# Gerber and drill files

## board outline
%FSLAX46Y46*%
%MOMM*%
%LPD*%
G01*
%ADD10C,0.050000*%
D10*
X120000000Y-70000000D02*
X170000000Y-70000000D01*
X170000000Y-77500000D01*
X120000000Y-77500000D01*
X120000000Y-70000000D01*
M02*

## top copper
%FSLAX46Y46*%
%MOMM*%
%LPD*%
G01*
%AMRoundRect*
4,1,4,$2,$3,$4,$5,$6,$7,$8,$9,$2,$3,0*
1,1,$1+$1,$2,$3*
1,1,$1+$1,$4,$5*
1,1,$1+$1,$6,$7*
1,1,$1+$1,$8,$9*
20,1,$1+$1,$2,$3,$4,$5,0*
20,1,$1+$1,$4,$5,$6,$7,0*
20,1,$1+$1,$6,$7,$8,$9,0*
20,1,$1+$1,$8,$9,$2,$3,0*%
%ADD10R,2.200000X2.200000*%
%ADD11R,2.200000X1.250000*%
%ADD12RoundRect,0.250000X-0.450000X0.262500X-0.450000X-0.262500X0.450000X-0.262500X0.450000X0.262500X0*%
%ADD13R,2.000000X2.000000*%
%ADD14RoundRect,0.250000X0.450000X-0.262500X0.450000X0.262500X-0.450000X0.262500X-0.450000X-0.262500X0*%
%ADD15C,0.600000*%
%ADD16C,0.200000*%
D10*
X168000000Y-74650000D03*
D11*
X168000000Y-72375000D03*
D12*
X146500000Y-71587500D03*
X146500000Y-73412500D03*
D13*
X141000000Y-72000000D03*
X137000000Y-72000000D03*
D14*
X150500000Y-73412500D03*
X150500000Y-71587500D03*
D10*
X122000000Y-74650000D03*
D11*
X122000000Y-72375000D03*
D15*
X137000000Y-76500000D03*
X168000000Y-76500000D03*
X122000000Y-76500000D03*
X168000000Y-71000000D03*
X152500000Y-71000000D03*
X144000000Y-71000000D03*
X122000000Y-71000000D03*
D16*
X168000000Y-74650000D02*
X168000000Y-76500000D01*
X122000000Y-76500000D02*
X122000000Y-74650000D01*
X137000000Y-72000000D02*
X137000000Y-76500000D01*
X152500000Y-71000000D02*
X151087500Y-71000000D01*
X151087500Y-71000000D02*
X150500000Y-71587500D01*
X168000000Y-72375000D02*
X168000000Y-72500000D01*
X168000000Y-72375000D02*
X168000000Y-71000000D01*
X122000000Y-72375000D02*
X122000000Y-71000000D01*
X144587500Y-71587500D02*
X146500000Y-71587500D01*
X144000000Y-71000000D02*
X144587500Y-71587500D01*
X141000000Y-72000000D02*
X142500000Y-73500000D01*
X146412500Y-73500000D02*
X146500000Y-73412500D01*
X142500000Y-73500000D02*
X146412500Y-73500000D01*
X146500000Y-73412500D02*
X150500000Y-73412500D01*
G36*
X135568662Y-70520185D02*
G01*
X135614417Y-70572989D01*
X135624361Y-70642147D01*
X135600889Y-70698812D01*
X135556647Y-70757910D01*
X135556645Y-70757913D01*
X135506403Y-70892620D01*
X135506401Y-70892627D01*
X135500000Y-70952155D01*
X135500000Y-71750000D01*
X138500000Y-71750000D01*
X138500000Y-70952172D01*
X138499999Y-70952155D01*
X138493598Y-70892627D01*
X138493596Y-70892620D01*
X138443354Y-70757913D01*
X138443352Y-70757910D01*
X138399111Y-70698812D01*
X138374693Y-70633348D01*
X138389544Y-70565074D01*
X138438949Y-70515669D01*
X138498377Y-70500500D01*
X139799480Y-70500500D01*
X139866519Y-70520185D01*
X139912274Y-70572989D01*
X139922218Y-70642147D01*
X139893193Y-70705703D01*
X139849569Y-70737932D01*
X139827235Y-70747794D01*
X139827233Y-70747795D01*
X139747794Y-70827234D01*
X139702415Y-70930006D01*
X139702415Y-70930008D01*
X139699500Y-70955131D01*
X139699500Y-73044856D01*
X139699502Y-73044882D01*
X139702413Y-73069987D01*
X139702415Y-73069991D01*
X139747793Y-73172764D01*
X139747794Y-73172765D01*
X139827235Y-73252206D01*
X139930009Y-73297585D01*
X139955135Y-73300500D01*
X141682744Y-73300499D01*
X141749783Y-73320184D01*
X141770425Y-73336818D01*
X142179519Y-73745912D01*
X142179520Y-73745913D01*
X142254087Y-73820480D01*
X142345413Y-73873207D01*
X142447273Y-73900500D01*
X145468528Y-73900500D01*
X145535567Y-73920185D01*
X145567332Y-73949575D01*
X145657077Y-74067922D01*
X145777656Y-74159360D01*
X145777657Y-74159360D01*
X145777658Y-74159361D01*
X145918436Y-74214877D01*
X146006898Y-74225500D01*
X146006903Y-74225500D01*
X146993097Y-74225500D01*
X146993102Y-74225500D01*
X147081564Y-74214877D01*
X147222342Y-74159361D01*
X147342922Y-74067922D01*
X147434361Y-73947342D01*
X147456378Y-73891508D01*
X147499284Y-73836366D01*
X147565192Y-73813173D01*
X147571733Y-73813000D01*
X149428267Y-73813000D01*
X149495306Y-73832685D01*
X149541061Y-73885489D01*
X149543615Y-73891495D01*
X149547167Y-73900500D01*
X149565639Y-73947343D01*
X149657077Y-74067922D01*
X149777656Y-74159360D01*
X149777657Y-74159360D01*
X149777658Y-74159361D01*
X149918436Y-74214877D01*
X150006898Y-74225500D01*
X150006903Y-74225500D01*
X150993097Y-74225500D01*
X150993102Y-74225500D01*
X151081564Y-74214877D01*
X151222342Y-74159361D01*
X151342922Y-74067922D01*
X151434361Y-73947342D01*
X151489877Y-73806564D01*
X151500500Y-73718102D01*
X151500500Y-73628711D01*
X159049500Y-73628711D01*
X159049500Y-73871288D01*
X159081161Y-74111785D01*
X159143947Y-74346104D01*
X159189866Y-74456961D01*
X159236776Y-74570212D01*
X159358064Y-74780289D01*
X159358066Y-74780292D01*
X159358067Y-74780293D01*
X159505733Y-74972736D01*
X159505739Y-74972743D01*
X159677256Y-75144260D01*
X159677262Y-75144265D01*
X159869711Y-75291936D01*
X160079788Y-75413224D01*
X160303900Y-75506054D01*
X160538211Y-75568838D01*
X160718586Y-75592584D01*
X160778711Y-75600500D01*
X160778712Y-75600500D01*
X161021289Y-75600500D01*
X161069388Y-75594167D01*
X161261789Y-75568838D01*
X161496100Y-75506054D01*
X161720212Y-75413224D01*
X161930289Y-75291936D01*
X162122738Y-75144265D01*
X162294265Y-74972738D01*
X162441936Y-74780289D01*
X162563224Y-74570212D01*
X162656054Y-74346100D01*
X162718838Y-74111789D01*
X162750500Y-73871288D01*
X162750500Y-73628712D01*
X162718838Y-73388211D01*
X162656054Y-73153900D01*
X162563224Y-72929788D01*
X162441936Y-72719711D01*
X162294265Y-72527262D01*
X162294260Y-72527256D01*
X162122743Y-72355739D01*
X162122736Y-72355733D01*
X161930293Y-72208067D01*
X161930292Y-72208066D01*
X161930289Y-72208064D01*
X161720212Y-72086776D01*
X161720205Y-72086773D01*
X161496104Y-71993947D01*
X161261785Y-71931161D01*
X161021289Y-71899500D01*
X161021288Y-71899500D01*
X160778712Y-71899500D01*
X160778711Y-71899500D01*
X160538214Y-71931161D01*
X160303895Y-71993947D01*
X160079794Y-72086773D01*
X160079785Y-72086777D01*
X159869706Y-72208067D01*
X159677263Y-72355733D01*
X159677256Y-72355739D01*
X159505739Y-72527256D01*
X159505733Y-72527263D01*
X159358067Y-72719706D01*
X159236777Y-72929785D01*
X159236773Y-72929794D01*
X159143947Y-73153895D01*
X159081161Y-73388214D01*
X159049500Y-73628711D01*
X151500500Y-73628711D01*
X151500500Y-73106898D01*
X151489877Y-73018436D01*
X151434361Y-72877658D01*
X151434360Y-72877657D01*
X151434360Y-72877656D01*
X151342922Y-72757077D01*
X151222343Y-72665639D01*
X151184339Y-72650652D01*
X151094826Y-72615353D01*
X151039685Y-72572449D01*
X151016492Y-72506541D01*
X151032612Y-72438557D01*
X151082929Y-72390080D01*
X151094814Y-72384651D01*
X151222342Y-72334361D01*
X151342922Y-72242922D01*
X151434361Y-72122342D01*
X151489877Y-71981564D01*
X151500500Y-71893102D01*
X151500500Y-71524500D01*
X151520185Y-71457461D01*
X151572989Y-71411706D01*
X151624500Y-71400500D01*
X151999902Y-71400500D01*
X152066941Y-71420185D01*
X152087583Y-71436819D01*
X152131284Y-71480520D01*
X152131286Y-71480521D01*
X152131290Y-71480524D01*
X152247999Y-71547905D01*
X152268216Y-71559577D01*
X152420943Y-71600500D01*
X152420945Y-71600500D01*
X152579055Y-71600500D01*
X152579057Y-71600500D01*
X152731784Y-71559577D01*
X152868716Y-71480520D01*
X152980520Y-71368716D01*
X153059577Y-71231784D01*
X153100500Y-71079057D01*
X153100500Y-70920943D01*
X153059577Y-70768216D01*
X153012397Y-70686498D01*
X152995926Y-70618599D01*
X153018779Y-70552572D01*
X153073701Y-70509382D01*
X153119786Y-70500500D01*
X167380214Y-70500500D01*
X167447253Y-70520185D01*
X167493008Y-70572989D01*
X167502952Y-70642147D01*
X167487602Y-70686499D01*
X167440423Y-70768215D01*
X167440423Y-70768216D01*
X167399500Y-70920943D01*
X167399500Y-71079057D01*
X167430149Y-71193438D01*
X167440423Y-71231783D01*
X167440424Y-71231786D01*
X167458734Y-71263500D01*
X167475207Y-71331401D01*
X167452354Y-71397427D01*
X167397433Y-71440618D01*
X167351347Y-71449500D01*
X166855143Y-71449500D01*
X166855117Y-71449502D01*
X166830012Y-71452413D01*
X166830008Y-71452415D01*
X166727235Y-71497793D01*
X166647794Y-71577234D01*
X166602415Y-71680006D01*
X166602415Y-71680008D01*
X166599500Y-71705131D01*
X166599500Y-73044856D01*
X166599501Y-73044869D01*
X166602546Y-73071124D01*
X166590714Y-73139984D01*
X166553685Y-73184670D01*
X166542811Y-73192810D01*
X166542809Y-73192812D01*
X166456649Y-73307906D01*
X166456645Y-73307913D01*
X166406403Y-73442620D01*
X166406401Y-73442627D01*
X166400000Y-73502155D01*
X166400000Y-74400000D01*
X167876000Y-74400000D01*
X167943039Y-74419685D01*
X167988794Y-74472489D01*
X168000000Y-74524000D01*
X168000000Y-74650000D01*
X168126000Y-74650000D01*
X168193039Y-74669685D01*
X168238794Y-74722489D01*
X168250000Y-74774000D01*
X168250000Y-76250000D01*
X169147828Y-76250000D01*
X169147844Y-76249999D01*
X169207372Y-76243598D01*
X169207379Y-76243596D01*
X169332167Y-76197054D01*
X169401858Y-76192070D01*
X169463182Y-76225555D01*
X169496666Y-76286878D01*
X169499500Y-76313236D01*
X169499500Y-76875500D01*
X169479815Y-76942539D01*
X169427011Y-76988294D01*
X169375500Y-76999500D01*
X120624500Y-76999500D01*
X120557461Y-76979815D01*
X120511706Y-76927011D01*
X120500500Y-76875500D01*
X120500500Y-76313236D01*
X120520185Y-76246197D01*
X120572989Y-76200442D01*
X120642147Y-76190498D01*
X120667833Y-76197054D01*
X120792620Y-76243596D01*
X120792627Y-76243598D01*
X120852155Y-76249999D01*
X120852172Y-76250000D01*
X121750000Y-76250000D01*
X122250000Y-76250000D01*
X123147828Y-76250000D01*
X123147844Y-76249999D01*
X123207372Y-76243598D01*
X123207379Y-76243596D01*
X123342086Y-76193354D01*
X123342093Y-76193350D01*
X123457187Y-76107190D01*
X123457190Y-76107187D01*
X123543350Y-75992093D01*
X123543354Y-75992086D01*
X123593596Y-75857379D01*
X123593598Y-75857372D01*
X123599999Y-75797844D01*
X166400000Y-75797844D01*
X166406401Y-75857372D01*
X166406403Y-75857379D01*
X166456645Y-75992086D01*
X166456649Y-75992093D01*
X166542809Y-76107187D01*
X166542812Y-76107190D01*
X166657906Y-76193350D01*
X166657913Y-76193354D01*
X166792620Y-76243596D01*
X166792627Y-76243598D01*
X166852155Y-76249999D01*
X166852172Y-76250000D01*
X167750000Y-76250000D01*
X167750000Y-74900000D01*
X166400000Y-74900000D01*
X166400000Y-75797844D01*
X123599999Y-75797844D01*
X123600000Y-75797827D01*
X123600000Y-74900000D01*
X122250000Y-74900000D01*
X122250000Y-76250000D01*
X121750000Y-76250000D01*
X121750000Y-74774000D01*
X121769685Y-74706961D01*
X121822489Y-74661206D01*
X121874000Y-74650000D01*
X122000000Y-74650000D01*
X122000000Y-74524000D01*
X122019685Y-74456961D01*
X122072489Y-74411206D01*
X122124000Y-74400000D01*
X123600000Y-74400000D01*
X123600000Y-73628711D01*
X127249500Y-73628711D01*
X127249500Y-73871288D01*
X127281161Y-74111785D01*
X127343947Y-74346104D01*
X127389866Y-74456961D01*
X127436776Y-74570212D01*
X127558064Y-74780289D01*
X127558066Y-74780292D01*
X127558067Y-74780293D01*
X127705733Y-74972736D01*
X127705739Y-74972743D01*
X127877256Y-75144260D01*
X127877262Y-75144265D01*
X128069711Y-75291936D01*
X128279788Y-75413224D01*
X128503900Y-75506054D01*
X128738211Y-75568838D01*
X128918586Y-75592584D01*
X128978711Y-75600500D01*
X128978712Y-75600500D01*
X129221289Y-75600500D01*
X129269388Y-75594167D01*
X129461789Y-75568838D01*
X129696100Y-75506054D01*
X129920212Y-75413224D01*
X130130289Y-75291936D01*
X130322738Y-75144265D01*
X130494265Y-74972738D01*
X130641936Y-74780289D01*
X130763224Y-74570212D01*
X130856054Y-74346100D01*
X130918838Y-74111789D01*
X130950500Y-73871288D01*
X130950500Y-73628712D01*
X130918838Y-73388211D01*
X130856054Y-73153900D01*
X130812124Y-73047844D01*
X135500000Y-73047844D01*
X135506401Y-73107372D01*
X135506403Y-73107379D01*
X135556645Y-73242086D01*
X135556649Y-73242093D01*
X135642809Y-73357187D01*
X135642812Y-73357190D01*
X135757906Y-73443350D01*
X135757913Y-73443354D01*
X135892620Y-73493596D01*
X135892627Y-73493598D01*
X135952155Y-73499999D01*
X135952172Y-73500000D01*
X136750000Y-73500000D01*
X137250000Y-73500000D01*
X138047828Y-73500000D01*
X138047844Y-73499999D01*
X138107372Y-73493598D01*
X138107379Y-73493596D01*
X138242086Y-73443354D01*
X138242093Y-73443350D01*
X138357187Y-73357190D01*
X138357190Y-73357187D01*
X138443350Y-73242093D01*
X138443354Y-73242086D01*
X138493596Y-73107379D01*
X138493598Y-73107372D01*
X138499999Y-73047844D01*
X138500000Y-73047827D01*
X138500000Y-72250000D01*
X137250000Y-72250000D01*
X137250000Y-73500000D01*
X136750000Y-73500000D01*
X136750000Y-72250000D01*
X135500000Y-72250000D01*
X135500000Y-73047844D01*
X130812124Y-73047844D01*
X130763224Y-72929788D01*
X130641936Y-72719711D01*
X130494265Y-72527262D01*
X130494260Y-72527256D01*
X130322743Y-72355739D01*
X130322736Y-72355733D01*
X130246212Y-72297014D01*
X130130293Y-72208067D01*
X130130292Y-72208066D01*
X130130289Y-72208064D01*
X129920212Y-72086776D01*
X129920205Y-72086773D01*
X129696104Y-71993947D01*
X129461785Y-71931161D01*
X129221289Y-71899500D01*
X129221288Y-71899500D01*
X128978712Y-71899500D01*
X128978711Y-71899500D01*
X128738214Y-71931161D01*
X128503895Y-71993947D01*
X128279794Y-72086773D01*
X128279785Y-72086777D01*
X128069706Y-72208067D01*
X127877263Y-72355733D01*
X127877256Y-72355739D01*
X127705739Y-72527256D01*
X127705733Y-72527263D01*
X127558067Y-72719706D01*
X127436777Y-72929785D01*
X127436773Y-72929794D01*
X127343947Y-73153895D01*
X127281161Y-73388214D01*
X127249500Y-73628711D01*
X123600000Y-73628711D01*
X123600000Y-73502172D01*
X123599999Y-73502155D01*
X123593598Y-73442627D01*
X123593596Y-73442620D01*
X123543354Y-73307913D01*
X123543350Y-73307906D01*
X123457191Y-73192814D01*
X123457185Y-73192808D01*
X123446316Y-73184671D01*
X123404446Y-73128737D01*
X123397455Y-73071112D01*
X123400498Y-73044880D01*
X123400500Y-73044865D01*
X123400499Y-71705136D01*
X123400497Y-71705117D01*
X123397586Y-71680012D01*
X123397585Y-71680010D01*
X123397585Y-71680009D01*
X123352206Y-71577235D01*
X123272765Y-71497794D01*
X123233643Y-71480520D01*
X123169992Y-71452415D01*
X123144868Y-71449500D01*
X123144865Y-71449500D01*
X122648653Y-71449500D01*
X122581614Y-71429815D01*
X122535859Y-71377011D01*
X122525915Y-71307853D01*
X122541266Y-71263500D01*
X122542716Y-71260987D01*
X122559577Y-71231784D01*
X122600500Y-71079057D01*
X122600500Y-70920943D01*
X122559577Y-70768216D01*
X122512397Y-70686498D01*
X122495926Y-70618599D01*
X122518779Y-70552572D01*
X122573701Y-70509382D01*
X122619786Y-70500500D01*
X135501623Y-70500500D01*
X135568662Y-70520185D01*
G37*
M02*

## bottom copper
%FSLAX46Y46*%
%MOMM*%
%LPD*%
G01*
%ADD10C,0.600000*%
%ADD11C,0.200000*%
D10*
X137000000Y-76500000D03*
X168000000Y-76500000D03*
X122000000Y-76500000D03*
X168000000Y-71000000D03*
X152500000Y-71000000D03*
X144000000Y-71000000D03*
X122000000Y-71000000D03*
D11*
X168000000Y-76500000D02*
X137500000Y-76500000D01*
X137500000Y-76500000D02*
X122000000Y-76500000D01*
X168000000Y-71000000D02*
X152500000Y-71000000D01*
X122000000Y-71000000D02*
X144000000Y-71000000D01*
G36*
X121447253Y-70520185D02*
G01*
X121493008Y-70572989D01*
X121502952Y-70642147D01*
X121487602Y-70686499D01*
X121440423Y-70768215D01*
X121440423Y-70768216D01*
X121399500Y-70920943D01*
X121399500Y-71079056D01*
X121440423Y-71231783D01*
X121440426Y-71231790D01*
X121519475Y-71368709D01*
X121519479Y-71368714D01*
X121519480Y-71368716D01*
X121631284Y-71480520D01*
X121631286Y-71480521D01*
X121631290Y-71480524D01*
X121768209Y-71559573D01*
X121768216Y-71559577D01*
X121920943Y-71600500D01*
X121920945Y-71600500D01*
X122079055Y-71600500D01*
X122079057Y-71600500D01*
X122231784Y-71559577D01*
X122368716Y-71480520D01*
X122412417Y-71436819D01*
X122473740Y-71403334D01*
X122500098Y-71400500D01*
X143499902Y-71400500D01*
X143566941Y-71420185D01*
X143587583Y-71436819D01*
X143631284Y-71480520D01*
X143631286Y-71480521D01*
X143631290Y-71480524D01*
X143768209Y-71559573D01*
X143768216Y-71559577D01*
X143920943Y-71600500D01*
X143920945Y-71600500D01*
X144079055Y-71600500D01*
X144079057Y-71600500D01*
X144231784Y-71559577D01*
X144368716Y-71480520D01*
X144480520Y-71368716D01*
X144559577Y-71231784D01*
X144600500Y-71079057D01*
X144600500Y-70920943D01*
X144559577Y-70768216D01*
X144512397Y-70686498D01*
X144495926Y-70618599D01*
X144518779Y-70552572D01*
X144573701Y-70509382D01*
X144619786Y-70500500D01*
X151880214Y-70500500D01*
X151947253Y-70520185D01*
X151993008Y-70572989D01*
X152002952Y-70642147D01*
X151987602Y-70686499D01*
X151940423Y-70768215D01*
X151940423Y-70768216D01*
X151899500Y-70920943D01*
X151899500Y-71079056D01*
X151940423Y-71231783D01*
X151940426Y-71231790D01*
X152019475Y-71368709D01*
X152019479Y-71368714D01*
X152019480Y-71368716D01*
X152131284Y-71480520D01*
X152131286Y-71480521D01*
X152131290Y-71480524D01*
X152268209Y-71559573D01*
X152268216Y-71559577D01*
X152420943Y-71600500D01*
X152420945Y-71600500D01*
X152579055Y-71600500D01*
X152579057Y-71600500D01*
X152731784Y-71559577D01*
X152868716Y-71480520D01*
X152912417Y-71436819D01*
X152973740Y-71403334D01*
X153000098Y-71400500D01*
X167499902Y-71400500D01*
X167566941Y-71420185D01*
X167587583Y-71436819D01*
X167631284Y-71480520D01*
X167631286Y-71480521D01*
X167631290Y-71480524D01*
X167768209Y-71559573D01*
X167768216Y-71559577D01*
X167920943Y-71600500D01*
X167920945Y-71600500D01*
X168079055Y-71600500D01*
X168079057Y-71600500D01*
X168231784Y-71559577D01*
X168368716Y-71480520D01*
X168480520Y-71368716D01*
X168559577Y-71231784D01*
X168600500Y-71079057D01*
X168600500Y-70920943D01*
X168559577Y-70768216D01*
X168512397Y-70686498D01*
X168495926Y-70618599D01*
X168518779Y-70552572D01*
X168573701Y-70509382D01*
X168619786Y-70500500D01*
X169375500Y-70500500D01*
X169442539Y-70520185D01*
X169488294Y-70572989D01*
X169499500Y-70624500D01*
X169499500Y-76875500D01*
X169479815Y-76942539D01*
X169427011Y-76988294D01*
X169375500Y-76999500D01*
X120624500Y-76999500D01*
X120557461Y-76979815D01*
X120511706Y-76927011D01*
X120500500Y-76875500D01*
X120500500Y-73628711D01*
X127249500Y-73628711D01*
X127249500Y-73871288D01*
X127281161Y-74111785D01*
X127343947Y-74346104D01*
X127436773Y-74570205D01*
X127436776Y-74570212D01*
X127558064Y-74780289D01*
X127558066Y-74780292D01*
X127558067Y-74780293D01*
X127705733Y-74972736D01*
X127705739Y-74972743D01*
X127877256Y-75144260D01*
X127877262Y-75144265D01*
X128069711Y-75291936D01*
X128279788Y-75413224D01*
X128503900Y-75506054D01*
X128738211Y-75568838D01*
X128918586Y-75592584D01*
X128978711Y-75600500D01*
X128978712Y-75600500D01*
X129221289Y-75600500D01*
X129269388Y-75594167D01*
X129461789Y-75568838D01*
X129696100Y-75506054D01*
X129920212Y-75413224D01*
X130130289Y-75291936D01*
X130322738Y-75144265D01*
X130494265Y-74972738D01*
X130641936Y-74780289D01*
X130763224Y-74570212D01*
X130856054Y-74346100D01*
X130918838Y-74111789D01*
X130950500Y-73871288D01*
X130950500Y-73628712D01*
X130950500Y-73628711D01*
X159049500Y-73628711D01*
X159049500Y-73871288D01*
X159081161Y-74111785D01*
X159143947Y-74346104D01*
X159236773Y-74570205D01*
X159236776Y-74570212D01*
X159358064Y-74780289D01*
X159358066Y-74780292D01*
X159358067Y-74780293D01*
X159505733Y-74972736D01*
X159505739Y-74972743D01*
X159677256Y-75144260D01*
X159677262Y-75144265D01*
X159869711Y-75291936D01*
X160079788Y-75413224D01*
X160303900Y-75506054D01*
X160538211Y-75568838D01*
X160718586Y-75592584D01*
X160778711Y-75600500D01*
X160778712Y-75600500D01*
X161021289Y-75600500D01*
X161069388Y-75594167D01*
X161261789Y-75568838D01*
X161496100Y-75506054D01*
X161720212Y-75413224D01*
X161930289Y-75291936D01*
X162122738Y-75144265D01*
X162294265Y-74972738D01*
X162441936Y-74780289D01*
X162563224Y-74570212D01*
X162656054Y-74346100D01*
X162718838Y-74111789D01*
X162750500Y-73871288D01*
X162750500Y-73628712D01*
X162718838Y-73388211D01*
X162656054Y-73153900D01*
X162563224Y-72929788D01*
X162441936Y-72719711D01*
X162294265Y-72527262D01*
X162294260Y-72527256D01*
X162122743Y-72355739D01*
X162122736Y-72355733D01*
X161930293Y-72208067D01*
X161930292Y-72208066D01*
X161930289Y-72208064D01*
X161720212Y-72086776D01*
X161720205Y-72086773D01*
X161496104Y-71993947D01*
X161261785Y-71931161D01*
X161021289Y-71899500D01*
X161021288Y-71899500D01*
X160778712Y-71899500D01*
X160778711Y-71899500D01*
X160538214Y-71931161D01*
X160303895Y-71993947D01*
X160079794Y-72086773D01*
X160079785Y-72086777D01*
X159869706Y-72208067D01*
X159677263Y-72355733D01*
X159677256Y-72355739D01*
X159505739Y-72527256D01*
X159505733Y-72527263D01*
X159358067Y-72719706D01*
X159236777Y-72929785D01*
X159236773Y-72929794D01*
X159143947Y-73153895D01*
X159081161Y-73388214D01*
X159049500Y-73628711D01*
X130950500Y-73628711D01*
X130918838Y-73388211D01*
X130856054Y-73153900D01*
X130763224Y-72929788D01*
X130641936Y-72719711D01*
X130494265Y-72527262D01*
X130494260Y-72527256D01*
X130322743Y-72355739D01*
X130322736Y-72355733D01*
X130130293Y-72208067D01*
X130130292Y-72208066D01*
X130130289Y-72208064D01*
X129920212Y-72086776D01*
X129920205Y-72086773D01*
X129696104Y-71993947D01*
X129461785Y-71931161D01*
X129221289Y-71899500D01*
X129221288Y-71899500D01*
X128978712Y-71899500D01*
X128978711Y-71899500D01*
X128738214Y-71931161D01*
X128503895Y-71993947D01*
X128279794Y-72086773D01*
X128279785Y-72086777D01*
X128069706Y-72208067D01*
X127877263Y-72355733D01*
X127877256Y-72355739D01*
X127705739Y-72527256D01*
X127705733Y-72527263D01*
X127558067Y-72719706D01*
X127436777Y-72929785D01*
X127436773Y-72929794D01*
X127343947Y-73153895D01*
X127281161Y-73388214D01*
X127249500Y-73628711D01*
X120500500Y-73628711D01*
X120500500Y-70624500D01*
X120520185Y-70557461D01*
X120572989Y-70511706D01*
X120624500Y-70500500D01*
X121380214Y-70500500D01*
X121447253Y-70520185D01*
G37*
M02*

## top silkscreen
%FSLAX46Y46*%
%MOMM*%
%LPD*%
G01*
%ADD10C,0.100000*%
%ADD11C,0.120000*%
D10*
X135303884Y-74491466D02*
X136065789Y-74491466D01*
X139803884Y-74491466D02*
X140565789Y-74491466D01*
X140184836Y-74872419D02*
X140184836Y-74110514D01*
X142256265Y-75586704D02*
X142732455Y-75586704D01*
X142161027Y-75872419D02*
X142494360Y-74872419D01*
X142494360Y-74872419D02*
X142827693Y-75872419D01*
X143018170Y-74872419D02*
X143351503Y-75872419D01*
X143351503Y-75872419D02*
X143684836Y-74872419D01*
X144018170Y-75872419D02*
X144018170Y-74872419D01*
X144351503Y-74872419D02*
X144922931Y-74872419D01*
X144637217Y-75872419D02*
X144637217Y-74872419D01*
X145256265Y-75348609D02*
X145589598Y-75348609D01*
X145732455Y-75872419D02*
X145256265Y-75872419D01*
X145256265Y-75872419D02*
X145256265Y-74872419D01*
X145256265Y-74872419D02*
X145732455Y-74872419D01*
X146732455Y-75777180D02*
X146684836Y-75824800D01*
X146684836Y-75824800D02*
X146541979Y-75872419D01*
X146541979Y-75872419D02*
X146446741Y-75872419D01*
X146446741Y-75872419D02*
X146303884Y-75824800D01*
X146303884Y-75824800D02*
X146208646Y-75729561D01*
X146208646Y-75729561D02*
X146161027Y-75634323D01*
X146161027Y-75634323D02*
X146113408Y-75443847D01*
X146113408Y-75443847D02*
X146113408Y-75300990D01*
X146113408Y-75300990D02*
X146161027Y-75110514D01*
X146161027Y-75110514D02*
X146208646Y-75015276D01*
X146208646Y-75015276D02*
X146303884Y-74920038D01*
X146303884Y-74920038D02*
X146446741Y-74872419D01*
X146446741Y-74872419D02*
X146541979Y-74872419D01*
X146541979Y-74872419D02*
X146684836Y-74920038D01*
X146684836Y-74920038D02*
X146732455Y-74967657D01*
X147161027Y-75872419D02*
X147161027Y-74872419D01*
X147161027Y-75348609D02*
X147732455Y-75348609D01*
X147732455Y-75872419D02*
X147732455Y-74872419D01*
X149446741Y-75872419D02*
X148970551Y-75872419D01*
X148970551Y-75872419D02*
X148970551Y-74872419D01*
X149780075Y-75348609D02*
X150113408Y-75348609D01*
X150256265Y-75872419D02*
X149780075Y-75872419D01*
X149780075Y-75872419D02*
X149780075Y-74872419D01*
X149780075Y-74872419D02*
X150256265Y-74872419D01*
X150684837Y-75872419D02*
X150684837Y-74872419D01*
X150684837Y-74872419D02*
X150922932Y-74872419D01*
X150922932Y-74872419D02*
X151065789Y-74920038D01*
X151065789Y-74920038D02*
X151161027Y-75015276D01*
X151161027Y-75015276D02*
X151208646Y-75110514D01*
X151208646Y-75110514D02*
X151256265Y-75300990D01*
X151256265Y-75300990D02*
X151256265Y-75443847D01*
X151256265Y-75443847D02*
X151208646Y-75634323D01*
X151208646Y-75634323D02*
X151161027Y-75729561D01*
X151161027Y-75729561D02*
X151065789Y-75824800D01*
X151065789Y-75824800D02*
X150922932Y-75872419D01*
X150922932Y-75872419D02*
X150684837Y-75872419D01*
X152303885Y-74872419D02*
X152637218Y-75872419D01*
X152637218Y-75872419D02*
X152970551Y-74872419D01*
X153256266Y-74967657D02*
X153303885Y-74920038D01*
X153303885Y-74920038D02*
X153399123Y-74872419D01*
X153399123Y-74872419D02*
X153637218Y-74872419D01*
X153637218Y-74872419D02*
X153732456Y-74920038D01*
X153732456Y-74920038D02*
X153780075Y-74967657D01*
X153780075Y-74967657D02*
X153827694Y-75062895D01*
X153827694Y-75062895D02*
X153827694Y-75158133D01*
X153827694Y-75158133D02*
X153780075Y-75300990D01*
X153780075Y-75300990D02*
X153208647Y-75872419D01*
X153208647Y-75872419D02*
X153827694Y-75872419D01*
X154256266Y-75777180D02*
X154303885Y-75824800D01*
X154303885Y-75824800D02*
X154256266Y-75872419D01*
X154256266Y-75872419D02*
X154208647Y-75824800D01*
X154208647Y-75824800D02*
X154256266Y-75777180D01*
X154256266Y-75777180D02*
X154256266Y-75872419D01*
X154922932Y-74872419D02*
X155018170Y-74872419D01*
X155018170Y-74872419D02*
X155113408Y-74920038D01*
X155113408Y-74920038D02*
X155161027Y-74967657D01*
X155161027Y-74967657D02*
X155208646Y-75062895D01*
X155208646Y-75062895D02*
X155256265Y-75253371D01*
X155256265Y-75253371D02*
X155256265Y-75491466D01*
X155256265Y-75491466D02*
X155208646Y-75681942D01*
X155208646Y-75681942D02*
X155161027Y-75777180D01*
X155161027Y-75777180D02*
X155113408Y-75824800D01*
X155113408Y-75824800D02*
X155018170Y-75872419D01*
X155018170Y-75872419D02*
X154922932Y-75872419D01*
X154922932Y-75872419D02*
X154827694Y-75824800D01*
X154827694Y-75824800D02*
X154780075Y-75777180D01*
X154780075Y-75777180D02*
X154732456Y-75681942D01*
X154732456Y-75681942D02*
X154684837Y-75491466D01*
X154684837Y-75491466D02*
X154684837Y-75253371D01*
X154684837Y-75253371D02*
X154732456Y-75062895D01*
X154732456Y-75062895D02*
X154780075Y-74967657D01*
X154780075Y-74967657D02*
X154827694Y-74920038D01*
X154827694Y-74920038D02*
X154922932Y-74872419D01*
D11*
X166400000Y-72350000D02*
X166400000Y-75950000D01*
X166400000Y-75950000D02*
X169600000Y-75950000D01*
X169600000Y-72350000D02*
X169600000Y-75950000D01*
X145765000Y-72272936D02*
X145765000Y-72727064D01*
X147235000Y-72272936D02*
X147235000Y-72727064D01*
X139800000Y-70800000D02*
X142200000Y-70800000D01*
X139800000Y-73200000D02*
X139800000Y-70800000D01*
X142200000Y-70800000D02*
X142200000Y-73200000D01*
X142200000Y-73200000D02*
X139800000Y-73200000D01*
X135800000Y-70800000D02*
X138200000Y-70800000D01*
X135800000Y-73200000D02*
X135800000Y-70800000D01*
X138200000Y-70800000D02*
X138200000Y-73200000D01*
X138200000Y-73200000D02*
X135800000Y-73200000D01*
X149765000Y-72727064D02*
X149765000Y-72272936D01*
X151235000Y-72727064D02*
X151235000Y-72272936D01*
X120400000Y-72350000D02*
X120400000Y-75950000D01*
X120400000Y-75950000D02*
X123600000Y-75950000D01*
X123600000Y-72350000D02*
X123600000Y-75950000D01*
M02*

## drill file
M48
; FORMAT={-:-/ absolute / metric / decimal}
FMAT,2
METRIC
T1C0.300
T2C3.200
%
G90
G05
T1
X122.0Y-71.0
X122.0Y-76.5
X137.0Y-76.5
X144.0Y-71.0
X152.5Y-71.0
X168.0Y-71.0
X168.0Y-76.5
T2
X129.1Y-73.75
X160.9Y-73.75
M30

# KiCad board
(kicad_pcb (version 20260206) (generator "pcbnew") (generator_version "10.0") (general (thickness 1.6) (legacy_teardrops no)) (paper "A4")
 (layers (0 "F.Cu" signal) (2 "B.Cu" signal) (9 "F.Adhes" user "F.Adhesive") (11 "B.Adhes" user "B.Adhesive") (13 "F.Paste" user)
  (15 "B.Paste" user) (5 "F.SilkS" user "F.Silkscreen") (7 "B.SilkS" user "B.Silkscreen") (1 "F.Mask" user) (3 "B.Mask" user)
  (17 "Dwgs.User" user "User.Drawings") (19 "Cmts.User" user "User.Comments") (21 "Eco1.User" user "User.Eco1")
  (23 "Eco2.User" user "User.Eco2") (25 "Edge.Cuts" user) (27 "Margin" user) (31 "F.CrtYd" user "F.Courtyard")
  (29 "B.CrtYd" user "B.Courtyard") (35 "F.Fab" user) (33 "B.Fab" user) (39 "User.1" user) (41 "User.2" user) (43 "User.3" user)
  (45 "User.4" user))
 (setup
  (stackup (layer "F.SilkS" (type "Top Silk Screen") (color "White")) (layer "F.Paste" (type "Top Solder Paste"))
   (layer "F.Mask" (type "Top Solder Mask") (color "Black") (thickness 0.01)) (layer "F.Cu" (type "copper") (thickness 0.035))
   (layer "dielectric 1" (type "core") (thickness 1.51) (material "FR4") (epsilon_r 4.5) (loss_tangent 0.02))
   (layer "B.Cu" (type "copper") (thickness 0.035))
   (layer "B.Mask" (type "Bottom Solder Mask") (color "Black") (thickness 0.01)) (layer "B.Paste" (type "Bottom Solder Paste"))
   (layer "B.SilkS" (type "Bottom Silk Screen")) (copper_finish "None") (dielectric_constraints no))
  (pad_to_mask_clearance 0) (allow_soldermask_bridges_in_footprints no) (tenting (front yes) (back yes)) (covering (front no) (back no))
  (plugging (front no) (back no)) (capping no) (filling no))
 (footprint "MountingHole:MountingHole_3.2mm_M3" (layer "F.Cu") (at 160.9 73.75)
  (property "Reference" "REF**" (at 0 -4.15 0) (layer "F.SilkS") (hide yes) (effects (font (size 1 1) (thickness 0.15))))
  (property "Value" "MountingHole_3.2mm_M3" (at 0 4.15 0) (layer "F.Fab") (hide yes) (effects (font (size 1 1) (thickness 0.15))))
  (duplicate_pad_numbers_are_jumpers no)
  (pad "" np_thru_hole circle (at 0 0) (size 3.2 3.2) (drill 3.2) (layers "*.Cu" "*.Mask")))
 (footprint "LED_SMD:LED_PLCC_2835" (layer "F.Cu") (at 168 73.75 90)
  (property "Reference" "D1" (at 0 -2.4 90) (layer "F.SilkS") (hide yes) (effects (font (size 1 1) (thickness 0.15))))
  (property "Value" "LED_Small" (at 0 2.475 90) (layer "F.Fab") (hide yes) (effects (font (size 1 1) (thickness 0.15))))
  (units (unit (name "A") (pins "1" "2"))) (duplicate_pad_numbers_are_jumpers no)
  (fp_line (start 1.4 -1.6) (end -2.2 -1.6) (stroke (width 0.12) (type solid)) (layer "F.SilkS"))
  (fp_line (start -2.2 -1.6) (end -2.2 1.6) (stroke (width 0.12) (type solid)) (layer "F.SilkS"))
  (fp_line (start 1.4 1.6) (end -2.2 1.6) (stroke (width 0.12) (type solid)) (layer "F.SilkS"))
  (pad "1" smd rect (at -0.9 0 90) (size 2.2 2.2) (layers "F.Cu" "F.Mask" "F.Paste") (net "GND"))
  (pad "2" smd rect (at 1.375 0 90) (size 1.25 2.2) (layers "F.Cu" "F.Mask" "F.Paste") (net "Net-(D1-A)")))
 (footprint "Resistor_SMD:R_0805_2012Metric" (layer "F.Cu") (at 146.5 72.5 -90)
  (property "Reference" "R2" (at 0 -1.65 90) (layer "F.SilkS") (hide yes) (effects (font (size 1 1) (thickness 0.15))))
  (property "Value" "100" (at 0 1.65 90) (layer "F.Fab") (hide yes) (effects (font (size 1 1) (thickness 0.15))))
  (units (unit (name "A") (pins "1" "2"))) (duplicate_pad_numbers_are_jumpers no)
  (fp_line (start -0.227064 0.735) (end 0.227064 0.735) (stroke (width 0.12) (type solid)) (layer "F.SilkS"))
  (fp_line (start -0.227064 -0.735) (end 0.227064 -0.735) (stroke (width 0.12) (type solid)) (layer "F.SilkS"))
  (pad "1" smd roundrect (at -0.9125 0 270) (size 1.025 1.4) (layers "F.Cu" "F.Mask" "F.Paste") (roundrect_rratio 0.243902)
   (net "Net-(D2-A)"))
  (pad "2" smd roundrect (at 0.9125 0 270) (size 1.025 1.4) (layers "F.Cu" "F.Mask" "F.Paste") (roundrect_rratio 0.243902)
   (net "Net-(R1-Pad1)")))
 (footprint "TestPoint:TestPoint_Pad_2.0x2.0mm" (layer "F.Cu") (at 141 72)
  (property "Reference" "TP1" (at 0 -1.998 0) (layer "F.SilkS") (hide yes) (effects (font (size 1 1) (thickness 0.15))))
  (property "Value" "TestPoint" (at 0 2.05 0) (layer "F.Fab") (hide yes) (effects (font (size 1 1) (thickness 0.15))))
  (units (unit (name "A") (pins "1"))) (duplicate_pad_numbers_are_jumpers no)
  (fp_line (start -1.2 -1.2) (end 1.2 -1.2) (stroke (width 0.12) (type solid)) (layer "F.SilkS"))
  (fp_line (start -1.2 1.2) (end -1.2 -1.2) (stroke (width 0.12) (type solid)) (layer "F.SilkS"))
  (fp_line (start 1.2 -1.2) (end 1.2 1.2) (stroke (width 0.12) (type solid)) (layer "F.SilkS"))
  (fp_line (start 1.2 1.2) (end -1.2 1.2) (stroke (width 0.12) (type solid)) (layer "F.SilkS"))
  (pad "1" smd rect (at 0 0) (size 2 2) (layers "F.Cu" "F.Mask") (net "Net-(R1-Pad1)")))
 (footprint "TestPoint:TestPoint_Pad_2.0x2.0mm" (layer "F.Cu") (at 137 72)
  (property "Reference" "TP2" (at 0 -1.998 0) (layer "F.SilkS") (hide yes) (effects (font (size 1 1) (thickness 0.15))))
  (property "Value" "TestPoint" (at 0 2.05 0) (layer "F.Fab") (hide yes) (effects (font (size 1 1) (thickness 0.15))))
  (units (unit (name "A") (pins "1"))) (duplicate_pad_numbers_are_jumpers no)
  (fp_line (start -1.2 -1.2) (end 1.2 -1.2) (stroke (width 0.12) (type solid)) (layer "F.SilkS"))
  (fp_line (start -1.2 1.2) (end -1.2 -1.2) (stroke (width 0.12) (type solid)) (layer "F.SilkS"))
  (fp_line (start 1.2 -1.2) (end 1.2 1.2) (stroke (width 0.12) (type solid)) (layer "F.SilkS"))
  (fp_line (start 1.2 1.2) (end -1.2 1.2) (stroke (width 0.12) (type solid)) (layer "F.SilkS"))
  (pad "1" smd rect (at 0 0) (size 2 2) (layers "F.Cu" "F.Mask") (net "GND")))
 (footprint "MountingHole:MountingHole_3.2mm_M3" (layer "F.Cu") (at 129.1 73.75)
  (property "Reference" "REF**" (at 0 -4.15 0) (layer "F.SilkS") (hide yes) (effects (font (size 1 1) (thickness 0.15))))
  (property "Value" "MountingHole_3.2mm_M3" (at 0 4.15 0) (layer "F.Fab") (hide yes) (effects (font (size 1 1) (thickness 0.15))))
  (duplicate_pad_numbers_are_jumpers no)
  (pad "" np_thru_hole circle (at 0 0) (size 3.2 3.2) (drill 3.2) (layers "*.Cu" "*.Mask")))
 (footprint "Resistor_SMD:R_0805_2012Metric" (layer "F.Cu") (at 150.5 72.5 90)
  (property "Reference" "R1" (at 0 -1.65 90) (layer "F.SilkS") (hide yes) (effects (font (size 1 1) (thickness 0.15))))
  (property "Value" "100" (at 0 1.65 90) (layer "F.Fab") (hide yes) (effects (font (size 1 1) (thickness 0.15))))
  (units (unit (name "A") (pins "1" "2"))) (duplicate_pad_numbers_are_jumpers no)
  (fp_line (start -0.227064 -0.735) (end 0.227064 -0.735) (stroke (width 0.12) (type solid)) (layer "F.SilkS"))
  (fp_line (start -0.227064 0.735) (end 0.227064 0.735) (stroke (width 0.12) (type solid)) (layer "F.SilkS"))
  (pad "1" smd roundrect (at -0.9125 0 90) (size 1.025 1.4) (layers "F.Cu" "F.Mask" "F.Paste") (roundrect_rratio 0.243902)
   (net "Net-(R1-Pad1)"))
  (pad "2" smd roundrect (at 0.9125 0 90) (size 1.025 1.4) (layers "F.Cu" "F.Mask" "F.Paste") (roundrect_rratio 0.243902) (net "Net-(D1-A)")))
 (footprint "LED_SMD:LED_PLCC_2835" (layer "F.Cu") (at 122 73.75 90)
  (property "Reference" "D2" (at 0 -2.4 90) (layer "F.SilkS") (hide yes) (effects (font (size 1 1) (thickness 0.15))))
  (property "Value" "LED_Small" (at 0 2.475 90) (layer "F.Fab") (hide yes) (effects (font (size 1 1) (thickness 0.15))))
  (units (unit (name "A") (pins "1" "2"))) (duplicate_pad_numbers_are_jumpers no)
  (fp_line (start 1.4 -1.6) (end -2.2 -1.6) (stroke (width 0.12) (type solid)) (layer "F.SilkS"))
  (fp_line (start -2.2 -1.6) (end -2.2 1.6) (stroke (width 0.12) (type solid)) (layer "F.SilkS"))
  (fp_line (start 1.4 1.6) (end -2.2 1.6) (stroke (width 0.12) (type solid)) (layer "F.SilkS"))
  (pad "1" smd rect (at -0.9 0 90) (size 2.2 2.2) (layers "F.Cu" "F.Mask" "F.Paste") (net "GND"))
  (pad "2" smd rect (at 1.375 0 90) (size 1.25 2.2) (layers "F.Cu" "F.Mask" "F.Paste") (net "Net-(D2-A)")))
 (gr_rect (start 120 70) (end 170 77.5) (stroke (width 0.05) (type default)) (fill no) (layer "Edge.Cuts"))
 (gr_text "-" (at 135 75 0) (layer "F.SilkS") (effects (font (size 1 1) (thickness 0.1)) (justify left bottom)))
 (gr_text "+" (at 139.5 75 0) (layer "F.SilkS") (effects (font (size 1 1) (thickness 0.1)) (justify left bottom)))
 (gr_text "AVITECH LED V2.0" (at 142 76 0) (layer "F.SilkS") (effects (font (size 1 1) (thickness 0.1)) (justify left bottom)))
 (segment (start 168 74.65) (end 168 76.5) (width 0.2) (layer "F.Cu") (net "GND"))
 (segment (start 122 76.5) (end 122 74.65) (width 0.2) (layer "F.Cu") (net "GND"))
 (segment (start 137 72) (end 137 76.5) (width 0.2) (layer "F.Cu") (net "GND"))
 (via (at 137 76.5) (size 0.6) (drill 0.3) (layers "F.Cu" "B.Cu") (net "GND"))
 (via (at 168 76.5) (size 0.6) (drill 0.3) (layers "F.Cu" "B.Cu") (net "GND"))
 (via (at 122 76.5) (size 0.6) (drill 0.3) (layers "F.Cu" "B.Cu") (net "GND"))
 (segment (start 168 76.5) (end 137.5 76.5) (width 0.2) (layer "B.Cu") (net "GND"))
 (segment (start 137.5 76.5) (end 122 76.5) (width 0.2) (layer "B.Cu") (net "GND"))
 (segment (start 152.5 71) (end 151.0875 71) (width 0.2) (layer "F.Cu") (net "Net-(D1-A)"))
 (segment (start 151.0875 71) (end 150.5 71.5875) (width 0.2) (layer "F.Cu") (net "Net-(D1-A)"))
 (segment (start 168 72.375) (end 168 72.5) (width 0.2) (layer "F.Cu") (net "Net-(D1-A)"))
 (segment (start 168 72.375) (end 168 71) (width 0.2) (layer "F.Cu") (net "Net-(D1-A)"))
 (via (at 168 71) (size 0.6) (drill 0.3) (layers "F.Cu" "B.Cu") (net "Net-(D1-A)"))
 (via (at 152.5 71) (size 0.6) (drill 0.3) (layers "F.Cu" "B.Cu") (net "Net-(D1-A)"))
 (segment (start 168 71) (end 152.5 71) (width 0.2) (layer "B.Cu") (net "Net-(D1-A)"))
 (segment (start 122 72.375) (end 122 71) (width 0.2) (layer "F.Cu") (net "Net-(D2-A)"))
 (segment (start 144.5875 71.5875) (end 146.5 71.5875) (width 0.2) (layer "F.Cu") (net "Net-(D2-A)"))
 (segment (start 144 71) (end 144.5875 71.5875) (width 0.2) (layer "F.Cu") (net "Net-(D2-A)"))
 (via (at 144 71) (size 0.6) (drill 0.3) (layers "F.Cu" "B.Cu") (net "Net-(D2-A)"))
 (via (at 122 71) (size 0.6) (drill 0.3) (layers "F.Cu" "B.Cu") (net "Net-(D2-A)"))
 (segment (start 122 71) (end 144 71) (width 0.2) (layer "B.Cu") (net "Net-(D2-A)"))
 (segment (start 141 72) (end 142.5 73.5) (width 0.2) (layer "F.Cu") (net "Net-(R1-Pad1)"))
 (segment (start 146.4125 73.5) (end 146.5 73.4125) (width 0.2) (layer "F.Cu") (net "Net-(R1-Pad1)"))
 (segment (start 142.5 73.5) (end 146.4125 73.5) (width 0.2) (layer "F.Cu") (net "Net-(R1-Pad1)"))
 (segment (start 146.5 73.4125) (end 150.5 73.4125) (width 0.2) (layer "F.Cu") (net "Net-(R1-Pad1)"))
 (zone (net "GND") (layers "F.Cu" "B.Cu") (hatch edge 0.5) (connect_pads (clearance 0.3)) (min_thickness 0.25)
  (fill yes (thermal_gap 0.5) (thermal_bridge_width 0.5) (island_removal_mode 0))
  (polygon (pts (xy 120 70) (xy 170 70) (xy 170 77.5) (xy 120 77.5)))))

